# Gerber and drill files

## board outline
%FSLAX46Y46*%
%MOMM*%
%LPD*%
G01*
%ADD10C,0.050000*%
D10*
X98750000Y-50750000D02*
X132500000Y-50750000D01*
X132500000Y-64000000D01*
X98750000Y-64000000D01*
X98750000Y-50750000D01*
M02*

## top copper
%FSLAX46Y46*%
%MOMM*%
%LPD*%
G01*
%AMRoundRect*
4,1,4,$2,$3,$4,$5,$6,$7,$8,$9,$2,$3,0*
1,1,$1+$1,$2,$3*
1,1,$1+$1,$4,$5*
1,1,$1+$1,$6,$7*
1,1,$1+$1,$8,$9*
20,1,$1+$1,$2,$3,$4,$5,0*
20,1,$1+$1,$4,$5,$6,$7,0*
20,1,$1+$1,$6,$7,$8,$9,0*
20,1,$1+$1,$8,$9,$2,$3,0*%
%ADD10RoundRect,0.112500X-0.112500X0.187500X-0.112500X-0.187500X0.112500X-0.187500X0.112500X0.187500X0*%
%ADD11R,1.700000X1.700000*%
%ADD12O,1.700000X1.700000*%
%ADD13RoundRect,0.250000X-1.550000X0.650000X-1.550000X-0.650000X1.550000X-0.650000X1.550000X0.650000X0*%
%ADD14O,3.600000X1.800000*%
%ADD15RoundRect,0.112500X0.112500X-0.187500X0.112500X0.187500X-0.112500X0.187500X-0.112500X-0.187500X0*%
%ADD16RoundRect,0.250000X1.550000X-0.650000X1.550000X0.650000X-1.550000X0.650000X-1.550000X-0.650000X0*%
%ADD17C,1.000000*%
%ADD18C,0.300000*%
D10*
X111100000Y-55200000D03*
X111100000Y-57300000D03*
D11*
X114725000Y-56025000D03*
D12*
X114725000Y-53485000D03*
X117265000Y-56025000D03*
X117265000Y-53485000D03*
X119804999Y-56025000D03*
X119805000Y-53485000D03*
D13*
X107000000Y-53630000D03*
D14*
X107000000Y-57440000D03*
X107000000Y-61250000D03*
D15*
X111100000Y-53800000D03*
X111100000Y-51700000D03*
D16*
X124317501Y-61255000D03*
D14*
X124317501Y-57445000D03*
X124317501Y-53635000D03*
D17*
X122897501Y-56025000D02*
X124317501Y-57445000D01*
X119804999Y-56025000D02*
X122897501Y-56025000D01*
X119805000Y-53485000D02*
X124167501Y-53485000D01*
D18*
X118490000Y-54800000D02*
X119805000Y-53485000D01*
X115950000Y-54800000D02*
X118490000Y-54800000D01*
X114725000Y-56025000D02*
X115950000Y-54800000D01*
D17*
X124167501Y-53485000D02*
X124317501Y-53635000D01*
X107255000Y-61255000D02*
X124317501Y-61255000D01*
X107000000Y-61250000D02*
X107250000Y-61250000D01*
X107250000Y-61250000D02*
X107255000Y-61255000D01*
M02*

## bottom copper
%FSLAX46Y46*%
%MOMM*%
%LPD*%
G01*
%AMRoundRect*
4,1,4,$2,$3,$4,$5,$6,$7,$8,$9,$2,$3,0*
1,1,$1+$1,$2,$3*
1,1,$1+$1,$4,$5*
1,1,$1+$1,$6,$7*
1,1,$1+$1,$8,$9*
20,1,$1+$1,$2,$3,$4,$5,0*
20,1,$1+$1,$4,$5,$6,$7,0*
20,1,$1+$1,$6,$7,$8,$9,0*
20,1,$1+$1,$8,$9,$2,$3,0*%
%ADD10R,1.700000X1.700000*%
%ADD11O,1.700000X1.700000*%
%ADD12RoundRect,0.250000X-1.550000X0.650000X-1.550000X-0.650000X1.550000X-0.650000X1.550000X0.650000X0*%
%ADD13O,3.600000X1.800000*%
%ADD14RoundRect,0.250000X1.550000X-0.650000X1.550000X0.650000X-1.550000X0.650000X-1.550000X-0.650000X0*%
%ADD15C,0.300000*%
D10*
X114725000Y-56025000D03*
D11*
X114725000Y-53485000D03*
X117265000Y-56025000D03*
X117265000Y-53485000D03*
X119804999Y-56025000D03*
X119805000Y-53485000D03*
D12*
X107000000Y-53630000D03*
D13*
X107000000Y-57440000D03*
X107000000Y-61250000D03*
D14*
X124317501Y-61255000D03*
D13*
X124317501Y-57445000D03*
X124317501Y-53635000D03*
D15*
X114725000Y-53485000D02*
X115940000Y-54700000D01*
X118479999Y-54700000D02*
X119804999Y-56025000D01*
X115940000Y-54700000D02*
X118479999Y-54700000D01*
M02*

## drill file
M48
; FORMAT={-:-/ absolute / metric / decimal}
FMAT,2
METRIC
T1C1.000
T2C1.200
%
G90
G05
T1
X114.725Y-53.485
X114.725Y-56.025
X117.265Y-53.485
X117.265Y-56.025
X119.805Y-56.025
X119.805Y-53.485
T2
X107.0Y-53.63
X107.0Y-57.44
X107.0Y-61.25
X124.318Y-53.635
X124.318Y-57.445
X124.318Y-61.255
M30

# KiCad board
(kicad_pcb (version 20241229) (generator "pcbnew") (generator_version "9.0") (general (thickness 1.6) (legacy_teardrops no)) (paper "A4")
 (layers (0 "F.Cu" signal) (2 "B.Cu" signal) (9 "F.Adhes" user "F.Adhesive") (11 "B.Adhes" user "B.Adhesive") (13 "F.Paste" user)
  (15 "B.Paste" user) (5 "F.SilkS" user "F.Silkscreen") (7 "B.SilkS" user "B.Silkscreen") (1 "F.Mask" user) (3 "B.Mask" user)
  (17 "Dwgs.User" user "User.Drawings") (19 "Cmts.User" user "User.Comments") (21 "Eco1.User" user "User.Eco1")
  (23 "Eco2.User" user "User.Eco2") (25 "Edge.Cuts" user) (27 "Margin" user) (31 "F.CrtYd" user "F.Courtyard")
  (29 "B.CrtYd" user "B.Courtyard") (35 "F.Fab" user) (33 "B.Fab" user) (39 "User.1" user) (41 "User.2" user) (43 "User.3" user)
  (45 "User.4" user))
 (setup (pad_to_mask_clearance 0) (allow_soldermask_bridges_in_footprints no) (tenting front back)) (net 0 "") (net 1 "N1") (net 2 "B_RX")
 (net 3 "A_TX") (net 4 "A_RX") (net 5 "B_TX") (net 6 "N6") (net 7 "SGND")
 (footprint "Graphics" (layer "F.Cu") (at 133.25 50.25)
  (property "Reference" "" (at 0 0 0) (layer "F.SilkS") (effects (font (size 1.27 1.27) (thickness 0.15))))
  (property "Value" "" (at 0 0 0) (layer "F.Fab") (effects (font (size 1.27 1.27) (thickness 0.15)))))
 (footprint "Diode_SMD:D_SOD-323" (layer "F.Cu") (at 111.1 56.25 -90)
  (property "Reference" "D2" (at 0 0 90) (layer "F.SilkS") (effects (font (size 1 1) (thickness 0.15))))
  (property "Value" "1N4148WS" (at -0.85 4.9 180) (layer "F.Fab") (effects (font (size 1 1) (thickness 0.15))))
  (pad "1" smd roundrect (at -1.05 0 270) (size 0.6 0.45) (layers "F.Cu" "F.Mask" "F.Paste") (roundrect_rratio 0.25) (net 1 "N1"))
  (pad "2" smd roundrect (at 1.05 0 270) (size 0.6 0.45) (layers "F.Cu" "F.Mask" "F.Paste") (roundrect_rratio 0.25) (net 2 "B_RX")))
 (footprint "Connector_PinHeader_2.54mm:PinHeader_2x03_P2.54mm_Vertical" (layer "F.Cu") (at 114.725 56.025 90)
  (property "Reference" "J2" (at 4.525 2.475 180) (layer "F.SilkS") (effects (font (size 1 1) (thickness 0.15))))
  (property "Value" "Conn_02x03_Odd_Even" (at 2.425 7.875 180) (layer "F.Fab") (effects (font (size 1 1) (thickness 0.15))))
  (pad "1" thru_hole rect (at 0 0 90) (size 1.7 1.7) (drill 1) (layers "*.Cu" "*.Mask") (remove_unused_layers no) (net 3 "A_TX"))
  (pad "2" thru_hole oval (at 2.54 0 90) (size 1.7 1.7) (drill 1) (layers "*.Cu" "*.Mask") (remove_unused_layers no) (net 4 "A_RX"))
  (pad "3" thru_hole oval (at 0 2.54 90) (size 1.7 1.7) (drill 1) (layers "*.Cu" "*.Mask") (remove_unused_layers no) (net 2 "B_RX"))
  (pad "4" thru_hole oval (at 2.54 2.54 90) (size 1.7 1.7) (drill 1) (layers "*.Cu" "*.Mask") (remove_unused_layers no) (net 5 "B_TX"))
  (pad "5" thru_hole oval (at 0 5.079999 90) (size 1.7 1.7) (drill 1) (layers "*.Cu" "*.Mask") (remove_unused_layers no) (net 4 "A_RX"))
  (pad "6" thru_hole oval (at 2.54 5.08 90) (size 1.7 1.7) (drill 1) (layers "*.Cu" "*.Mask") (remove_unused_layers no) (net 3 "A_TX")))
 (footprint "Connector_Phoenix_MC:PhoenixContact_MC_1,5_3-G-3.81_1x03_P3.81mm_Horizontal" (layer "F.Cu") (at 107 53.63 -90)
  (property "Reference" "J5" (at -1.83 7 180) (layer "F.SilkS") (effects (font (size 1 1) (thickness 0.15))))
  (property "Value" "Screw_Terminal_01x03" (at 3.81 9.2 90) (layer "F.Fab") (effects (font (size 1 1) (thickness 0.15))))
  (pad "1" thru_hole roundrect (at 0 0 270) (size 1.8 3.6) (drill 1.2) (layers "*.Cu" "*.Mask") (remove_unused_layers no)
   (roundrect_rratio 0.138889) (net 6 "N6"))
  (pad "2" thru_hole oval (at 3.81 0 270) (size 1.8 3.6) (drill 1.2) (layers "*.Cu" "*.Mask") (remove_unused_layers no) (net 1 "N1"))
  (pad "3" thru_hole oval (at 7.62 0 270) (size 1.8 3.6) (drill 1.2) (layers "*.Cu" "*.Mask") (remove_unused_layers no) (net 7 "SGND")))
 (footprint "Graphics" (layer "F.Cu") (at 133.25 50.25)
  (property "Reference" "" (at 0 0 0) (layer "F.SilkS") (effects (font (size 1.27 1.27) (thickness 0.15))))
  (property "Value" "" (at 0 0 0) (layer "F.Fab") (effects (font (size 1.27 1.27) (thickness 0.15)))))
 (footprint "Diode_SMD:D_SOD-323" (layer "F.Cu") (at 111.1 52.75 90)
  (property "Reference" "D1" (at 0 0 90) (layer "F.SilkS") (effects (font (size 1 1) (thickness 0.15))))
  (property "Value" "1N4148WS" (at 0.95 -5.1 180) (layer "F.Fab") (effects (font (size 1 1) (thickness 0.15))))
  (pad "1" smd roundrect (at -1.05 0 90) (size 0.6 0.45) (layers "F.Cu" "F.Mask" "F.Paste") (roundrect_rratio 0.25) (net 6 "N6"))
  (pad "2" smd roundrect (at 1.05 0 90) (size 0.6 0.45) (layers "F.Cu" "F.Mask" "F.Paste") (roundrect_rratio 0.25) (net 5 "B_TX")))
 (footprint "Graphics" (layer "F.Cu") (at 133.25 50.25)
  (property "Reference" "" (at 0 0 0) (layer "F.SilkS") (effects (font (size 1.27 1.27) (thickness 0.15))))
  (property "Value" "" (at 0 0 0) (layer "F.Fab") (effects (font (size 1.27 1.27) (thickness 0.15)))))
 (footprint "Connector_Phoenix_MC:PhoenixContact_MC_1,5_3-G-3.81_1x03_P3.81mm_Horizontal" (layer "F.Cu") (at 124.317501 61.255 90)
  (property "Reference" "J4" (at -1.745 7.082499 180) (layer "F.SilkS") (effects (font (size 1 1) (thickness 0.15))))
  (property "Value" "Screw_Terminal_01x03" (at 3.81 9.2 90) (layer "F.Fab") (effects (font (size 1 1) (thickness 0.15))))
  (pad "1" thru_hole roundrect (at 0 0 90) (size 1.8 3.6) (drill 1.2) (layers "*.Cu" "*.Mask") (remove_unused_layers no)
   (roundrect_rratio 0.138889) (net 7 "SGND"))
  (pad "2" thru_hole oval (at 3.81 0 90) (size 1.8 3.6) (drill 1.2) (layers "*.Cu" "*.Mask") (remove_unused_layers no) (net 4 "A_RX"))
  (pad "3" thru_hole oval (at 7.62 0 90) (size 1.8 3.6) (drill 1.2) (layers "*.Cu" "*.Mask") (remove_unused_layers no) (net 3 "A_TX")))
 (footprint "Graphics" (layer "F.Cu") (at 133.25 50.25)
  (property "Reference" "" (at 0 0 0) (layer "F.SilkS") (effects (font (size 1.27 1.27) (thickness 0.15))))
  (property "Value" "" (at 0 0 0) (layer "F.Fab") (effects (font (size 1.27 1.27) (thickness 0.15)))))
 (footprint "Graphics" (layer "B.Cu") (at 132.3905 50.909 180)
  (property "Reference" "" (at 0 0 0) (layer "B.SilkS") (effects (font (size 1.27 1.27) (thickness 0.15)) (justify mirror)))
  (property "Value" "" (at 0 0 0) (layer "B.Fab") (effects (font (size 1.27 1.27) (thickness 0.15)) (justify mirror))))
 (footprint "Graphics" (layer "B.Cu") (at 133.25 50.25)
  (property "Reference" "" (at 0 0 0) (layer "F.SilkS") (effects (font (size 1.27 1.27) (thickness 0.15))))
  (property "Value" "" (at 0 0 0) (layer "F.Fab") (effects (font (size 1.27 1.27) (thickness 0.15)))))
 (gr_rect (start 98.75 50.75) (end 132.5 64) (stroke (width 0.05) (type default)) (fill no) (layer "Edge.Cuts"))
 (segment (start 122.897501 56.025) (end 124.317501 57.445) (width 1) (layer "F.Cu") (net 4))
 (segment (start 119.804999 56.025) (end 122.897501 56.025) (width 1) (layer "F.Cu") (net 4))
 (segment (start 114.725 53.485) (end 115.94 54.7) (width 0.3) (layer "B.Cu") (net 4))
 (segment (start 118.479999 54.7) (end 119.804999 56.025) (width 0.3) (layer "B.Cu") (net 4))
 (segment (start 115.94 54.7) (end 118.479999 54.7) (width 0.3) (layer "B.Cu") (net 4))
 (segment (start 119.805 53.485) (end 124.167501 53.485) (width 1) (layer "F.Cu") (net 3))
 (segment (start 118.49 54.8) (end 119.805 53.485) (width 0.3) (layer "F.Cu") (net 3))
 (segment (start 115.95 54.8) (end 118.49 54.8) (width 0.3) (layer "F.Cu") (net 3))
 (segment (start 114.725 56.025) (end 115.95 54.8) (width 0.3) (layer "F.Cu") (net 3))
 (segment (start 124.167501 53.485) (end 124.317501 53.635) (width 1) (layer "F.Cu") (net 3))
 (segment (start 107.255 61.255) (end 124.317501 61.255) (width 1) (layer "F.Cu") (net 7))
 (segment (start 107 61.25) (end 107.25 61.25) (width 1) (layer "F.Cu") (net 7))
 (segment (start 107.25 61.25) (end 107.255 61.255) (width 1) (layer "F.Cu") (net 7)))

